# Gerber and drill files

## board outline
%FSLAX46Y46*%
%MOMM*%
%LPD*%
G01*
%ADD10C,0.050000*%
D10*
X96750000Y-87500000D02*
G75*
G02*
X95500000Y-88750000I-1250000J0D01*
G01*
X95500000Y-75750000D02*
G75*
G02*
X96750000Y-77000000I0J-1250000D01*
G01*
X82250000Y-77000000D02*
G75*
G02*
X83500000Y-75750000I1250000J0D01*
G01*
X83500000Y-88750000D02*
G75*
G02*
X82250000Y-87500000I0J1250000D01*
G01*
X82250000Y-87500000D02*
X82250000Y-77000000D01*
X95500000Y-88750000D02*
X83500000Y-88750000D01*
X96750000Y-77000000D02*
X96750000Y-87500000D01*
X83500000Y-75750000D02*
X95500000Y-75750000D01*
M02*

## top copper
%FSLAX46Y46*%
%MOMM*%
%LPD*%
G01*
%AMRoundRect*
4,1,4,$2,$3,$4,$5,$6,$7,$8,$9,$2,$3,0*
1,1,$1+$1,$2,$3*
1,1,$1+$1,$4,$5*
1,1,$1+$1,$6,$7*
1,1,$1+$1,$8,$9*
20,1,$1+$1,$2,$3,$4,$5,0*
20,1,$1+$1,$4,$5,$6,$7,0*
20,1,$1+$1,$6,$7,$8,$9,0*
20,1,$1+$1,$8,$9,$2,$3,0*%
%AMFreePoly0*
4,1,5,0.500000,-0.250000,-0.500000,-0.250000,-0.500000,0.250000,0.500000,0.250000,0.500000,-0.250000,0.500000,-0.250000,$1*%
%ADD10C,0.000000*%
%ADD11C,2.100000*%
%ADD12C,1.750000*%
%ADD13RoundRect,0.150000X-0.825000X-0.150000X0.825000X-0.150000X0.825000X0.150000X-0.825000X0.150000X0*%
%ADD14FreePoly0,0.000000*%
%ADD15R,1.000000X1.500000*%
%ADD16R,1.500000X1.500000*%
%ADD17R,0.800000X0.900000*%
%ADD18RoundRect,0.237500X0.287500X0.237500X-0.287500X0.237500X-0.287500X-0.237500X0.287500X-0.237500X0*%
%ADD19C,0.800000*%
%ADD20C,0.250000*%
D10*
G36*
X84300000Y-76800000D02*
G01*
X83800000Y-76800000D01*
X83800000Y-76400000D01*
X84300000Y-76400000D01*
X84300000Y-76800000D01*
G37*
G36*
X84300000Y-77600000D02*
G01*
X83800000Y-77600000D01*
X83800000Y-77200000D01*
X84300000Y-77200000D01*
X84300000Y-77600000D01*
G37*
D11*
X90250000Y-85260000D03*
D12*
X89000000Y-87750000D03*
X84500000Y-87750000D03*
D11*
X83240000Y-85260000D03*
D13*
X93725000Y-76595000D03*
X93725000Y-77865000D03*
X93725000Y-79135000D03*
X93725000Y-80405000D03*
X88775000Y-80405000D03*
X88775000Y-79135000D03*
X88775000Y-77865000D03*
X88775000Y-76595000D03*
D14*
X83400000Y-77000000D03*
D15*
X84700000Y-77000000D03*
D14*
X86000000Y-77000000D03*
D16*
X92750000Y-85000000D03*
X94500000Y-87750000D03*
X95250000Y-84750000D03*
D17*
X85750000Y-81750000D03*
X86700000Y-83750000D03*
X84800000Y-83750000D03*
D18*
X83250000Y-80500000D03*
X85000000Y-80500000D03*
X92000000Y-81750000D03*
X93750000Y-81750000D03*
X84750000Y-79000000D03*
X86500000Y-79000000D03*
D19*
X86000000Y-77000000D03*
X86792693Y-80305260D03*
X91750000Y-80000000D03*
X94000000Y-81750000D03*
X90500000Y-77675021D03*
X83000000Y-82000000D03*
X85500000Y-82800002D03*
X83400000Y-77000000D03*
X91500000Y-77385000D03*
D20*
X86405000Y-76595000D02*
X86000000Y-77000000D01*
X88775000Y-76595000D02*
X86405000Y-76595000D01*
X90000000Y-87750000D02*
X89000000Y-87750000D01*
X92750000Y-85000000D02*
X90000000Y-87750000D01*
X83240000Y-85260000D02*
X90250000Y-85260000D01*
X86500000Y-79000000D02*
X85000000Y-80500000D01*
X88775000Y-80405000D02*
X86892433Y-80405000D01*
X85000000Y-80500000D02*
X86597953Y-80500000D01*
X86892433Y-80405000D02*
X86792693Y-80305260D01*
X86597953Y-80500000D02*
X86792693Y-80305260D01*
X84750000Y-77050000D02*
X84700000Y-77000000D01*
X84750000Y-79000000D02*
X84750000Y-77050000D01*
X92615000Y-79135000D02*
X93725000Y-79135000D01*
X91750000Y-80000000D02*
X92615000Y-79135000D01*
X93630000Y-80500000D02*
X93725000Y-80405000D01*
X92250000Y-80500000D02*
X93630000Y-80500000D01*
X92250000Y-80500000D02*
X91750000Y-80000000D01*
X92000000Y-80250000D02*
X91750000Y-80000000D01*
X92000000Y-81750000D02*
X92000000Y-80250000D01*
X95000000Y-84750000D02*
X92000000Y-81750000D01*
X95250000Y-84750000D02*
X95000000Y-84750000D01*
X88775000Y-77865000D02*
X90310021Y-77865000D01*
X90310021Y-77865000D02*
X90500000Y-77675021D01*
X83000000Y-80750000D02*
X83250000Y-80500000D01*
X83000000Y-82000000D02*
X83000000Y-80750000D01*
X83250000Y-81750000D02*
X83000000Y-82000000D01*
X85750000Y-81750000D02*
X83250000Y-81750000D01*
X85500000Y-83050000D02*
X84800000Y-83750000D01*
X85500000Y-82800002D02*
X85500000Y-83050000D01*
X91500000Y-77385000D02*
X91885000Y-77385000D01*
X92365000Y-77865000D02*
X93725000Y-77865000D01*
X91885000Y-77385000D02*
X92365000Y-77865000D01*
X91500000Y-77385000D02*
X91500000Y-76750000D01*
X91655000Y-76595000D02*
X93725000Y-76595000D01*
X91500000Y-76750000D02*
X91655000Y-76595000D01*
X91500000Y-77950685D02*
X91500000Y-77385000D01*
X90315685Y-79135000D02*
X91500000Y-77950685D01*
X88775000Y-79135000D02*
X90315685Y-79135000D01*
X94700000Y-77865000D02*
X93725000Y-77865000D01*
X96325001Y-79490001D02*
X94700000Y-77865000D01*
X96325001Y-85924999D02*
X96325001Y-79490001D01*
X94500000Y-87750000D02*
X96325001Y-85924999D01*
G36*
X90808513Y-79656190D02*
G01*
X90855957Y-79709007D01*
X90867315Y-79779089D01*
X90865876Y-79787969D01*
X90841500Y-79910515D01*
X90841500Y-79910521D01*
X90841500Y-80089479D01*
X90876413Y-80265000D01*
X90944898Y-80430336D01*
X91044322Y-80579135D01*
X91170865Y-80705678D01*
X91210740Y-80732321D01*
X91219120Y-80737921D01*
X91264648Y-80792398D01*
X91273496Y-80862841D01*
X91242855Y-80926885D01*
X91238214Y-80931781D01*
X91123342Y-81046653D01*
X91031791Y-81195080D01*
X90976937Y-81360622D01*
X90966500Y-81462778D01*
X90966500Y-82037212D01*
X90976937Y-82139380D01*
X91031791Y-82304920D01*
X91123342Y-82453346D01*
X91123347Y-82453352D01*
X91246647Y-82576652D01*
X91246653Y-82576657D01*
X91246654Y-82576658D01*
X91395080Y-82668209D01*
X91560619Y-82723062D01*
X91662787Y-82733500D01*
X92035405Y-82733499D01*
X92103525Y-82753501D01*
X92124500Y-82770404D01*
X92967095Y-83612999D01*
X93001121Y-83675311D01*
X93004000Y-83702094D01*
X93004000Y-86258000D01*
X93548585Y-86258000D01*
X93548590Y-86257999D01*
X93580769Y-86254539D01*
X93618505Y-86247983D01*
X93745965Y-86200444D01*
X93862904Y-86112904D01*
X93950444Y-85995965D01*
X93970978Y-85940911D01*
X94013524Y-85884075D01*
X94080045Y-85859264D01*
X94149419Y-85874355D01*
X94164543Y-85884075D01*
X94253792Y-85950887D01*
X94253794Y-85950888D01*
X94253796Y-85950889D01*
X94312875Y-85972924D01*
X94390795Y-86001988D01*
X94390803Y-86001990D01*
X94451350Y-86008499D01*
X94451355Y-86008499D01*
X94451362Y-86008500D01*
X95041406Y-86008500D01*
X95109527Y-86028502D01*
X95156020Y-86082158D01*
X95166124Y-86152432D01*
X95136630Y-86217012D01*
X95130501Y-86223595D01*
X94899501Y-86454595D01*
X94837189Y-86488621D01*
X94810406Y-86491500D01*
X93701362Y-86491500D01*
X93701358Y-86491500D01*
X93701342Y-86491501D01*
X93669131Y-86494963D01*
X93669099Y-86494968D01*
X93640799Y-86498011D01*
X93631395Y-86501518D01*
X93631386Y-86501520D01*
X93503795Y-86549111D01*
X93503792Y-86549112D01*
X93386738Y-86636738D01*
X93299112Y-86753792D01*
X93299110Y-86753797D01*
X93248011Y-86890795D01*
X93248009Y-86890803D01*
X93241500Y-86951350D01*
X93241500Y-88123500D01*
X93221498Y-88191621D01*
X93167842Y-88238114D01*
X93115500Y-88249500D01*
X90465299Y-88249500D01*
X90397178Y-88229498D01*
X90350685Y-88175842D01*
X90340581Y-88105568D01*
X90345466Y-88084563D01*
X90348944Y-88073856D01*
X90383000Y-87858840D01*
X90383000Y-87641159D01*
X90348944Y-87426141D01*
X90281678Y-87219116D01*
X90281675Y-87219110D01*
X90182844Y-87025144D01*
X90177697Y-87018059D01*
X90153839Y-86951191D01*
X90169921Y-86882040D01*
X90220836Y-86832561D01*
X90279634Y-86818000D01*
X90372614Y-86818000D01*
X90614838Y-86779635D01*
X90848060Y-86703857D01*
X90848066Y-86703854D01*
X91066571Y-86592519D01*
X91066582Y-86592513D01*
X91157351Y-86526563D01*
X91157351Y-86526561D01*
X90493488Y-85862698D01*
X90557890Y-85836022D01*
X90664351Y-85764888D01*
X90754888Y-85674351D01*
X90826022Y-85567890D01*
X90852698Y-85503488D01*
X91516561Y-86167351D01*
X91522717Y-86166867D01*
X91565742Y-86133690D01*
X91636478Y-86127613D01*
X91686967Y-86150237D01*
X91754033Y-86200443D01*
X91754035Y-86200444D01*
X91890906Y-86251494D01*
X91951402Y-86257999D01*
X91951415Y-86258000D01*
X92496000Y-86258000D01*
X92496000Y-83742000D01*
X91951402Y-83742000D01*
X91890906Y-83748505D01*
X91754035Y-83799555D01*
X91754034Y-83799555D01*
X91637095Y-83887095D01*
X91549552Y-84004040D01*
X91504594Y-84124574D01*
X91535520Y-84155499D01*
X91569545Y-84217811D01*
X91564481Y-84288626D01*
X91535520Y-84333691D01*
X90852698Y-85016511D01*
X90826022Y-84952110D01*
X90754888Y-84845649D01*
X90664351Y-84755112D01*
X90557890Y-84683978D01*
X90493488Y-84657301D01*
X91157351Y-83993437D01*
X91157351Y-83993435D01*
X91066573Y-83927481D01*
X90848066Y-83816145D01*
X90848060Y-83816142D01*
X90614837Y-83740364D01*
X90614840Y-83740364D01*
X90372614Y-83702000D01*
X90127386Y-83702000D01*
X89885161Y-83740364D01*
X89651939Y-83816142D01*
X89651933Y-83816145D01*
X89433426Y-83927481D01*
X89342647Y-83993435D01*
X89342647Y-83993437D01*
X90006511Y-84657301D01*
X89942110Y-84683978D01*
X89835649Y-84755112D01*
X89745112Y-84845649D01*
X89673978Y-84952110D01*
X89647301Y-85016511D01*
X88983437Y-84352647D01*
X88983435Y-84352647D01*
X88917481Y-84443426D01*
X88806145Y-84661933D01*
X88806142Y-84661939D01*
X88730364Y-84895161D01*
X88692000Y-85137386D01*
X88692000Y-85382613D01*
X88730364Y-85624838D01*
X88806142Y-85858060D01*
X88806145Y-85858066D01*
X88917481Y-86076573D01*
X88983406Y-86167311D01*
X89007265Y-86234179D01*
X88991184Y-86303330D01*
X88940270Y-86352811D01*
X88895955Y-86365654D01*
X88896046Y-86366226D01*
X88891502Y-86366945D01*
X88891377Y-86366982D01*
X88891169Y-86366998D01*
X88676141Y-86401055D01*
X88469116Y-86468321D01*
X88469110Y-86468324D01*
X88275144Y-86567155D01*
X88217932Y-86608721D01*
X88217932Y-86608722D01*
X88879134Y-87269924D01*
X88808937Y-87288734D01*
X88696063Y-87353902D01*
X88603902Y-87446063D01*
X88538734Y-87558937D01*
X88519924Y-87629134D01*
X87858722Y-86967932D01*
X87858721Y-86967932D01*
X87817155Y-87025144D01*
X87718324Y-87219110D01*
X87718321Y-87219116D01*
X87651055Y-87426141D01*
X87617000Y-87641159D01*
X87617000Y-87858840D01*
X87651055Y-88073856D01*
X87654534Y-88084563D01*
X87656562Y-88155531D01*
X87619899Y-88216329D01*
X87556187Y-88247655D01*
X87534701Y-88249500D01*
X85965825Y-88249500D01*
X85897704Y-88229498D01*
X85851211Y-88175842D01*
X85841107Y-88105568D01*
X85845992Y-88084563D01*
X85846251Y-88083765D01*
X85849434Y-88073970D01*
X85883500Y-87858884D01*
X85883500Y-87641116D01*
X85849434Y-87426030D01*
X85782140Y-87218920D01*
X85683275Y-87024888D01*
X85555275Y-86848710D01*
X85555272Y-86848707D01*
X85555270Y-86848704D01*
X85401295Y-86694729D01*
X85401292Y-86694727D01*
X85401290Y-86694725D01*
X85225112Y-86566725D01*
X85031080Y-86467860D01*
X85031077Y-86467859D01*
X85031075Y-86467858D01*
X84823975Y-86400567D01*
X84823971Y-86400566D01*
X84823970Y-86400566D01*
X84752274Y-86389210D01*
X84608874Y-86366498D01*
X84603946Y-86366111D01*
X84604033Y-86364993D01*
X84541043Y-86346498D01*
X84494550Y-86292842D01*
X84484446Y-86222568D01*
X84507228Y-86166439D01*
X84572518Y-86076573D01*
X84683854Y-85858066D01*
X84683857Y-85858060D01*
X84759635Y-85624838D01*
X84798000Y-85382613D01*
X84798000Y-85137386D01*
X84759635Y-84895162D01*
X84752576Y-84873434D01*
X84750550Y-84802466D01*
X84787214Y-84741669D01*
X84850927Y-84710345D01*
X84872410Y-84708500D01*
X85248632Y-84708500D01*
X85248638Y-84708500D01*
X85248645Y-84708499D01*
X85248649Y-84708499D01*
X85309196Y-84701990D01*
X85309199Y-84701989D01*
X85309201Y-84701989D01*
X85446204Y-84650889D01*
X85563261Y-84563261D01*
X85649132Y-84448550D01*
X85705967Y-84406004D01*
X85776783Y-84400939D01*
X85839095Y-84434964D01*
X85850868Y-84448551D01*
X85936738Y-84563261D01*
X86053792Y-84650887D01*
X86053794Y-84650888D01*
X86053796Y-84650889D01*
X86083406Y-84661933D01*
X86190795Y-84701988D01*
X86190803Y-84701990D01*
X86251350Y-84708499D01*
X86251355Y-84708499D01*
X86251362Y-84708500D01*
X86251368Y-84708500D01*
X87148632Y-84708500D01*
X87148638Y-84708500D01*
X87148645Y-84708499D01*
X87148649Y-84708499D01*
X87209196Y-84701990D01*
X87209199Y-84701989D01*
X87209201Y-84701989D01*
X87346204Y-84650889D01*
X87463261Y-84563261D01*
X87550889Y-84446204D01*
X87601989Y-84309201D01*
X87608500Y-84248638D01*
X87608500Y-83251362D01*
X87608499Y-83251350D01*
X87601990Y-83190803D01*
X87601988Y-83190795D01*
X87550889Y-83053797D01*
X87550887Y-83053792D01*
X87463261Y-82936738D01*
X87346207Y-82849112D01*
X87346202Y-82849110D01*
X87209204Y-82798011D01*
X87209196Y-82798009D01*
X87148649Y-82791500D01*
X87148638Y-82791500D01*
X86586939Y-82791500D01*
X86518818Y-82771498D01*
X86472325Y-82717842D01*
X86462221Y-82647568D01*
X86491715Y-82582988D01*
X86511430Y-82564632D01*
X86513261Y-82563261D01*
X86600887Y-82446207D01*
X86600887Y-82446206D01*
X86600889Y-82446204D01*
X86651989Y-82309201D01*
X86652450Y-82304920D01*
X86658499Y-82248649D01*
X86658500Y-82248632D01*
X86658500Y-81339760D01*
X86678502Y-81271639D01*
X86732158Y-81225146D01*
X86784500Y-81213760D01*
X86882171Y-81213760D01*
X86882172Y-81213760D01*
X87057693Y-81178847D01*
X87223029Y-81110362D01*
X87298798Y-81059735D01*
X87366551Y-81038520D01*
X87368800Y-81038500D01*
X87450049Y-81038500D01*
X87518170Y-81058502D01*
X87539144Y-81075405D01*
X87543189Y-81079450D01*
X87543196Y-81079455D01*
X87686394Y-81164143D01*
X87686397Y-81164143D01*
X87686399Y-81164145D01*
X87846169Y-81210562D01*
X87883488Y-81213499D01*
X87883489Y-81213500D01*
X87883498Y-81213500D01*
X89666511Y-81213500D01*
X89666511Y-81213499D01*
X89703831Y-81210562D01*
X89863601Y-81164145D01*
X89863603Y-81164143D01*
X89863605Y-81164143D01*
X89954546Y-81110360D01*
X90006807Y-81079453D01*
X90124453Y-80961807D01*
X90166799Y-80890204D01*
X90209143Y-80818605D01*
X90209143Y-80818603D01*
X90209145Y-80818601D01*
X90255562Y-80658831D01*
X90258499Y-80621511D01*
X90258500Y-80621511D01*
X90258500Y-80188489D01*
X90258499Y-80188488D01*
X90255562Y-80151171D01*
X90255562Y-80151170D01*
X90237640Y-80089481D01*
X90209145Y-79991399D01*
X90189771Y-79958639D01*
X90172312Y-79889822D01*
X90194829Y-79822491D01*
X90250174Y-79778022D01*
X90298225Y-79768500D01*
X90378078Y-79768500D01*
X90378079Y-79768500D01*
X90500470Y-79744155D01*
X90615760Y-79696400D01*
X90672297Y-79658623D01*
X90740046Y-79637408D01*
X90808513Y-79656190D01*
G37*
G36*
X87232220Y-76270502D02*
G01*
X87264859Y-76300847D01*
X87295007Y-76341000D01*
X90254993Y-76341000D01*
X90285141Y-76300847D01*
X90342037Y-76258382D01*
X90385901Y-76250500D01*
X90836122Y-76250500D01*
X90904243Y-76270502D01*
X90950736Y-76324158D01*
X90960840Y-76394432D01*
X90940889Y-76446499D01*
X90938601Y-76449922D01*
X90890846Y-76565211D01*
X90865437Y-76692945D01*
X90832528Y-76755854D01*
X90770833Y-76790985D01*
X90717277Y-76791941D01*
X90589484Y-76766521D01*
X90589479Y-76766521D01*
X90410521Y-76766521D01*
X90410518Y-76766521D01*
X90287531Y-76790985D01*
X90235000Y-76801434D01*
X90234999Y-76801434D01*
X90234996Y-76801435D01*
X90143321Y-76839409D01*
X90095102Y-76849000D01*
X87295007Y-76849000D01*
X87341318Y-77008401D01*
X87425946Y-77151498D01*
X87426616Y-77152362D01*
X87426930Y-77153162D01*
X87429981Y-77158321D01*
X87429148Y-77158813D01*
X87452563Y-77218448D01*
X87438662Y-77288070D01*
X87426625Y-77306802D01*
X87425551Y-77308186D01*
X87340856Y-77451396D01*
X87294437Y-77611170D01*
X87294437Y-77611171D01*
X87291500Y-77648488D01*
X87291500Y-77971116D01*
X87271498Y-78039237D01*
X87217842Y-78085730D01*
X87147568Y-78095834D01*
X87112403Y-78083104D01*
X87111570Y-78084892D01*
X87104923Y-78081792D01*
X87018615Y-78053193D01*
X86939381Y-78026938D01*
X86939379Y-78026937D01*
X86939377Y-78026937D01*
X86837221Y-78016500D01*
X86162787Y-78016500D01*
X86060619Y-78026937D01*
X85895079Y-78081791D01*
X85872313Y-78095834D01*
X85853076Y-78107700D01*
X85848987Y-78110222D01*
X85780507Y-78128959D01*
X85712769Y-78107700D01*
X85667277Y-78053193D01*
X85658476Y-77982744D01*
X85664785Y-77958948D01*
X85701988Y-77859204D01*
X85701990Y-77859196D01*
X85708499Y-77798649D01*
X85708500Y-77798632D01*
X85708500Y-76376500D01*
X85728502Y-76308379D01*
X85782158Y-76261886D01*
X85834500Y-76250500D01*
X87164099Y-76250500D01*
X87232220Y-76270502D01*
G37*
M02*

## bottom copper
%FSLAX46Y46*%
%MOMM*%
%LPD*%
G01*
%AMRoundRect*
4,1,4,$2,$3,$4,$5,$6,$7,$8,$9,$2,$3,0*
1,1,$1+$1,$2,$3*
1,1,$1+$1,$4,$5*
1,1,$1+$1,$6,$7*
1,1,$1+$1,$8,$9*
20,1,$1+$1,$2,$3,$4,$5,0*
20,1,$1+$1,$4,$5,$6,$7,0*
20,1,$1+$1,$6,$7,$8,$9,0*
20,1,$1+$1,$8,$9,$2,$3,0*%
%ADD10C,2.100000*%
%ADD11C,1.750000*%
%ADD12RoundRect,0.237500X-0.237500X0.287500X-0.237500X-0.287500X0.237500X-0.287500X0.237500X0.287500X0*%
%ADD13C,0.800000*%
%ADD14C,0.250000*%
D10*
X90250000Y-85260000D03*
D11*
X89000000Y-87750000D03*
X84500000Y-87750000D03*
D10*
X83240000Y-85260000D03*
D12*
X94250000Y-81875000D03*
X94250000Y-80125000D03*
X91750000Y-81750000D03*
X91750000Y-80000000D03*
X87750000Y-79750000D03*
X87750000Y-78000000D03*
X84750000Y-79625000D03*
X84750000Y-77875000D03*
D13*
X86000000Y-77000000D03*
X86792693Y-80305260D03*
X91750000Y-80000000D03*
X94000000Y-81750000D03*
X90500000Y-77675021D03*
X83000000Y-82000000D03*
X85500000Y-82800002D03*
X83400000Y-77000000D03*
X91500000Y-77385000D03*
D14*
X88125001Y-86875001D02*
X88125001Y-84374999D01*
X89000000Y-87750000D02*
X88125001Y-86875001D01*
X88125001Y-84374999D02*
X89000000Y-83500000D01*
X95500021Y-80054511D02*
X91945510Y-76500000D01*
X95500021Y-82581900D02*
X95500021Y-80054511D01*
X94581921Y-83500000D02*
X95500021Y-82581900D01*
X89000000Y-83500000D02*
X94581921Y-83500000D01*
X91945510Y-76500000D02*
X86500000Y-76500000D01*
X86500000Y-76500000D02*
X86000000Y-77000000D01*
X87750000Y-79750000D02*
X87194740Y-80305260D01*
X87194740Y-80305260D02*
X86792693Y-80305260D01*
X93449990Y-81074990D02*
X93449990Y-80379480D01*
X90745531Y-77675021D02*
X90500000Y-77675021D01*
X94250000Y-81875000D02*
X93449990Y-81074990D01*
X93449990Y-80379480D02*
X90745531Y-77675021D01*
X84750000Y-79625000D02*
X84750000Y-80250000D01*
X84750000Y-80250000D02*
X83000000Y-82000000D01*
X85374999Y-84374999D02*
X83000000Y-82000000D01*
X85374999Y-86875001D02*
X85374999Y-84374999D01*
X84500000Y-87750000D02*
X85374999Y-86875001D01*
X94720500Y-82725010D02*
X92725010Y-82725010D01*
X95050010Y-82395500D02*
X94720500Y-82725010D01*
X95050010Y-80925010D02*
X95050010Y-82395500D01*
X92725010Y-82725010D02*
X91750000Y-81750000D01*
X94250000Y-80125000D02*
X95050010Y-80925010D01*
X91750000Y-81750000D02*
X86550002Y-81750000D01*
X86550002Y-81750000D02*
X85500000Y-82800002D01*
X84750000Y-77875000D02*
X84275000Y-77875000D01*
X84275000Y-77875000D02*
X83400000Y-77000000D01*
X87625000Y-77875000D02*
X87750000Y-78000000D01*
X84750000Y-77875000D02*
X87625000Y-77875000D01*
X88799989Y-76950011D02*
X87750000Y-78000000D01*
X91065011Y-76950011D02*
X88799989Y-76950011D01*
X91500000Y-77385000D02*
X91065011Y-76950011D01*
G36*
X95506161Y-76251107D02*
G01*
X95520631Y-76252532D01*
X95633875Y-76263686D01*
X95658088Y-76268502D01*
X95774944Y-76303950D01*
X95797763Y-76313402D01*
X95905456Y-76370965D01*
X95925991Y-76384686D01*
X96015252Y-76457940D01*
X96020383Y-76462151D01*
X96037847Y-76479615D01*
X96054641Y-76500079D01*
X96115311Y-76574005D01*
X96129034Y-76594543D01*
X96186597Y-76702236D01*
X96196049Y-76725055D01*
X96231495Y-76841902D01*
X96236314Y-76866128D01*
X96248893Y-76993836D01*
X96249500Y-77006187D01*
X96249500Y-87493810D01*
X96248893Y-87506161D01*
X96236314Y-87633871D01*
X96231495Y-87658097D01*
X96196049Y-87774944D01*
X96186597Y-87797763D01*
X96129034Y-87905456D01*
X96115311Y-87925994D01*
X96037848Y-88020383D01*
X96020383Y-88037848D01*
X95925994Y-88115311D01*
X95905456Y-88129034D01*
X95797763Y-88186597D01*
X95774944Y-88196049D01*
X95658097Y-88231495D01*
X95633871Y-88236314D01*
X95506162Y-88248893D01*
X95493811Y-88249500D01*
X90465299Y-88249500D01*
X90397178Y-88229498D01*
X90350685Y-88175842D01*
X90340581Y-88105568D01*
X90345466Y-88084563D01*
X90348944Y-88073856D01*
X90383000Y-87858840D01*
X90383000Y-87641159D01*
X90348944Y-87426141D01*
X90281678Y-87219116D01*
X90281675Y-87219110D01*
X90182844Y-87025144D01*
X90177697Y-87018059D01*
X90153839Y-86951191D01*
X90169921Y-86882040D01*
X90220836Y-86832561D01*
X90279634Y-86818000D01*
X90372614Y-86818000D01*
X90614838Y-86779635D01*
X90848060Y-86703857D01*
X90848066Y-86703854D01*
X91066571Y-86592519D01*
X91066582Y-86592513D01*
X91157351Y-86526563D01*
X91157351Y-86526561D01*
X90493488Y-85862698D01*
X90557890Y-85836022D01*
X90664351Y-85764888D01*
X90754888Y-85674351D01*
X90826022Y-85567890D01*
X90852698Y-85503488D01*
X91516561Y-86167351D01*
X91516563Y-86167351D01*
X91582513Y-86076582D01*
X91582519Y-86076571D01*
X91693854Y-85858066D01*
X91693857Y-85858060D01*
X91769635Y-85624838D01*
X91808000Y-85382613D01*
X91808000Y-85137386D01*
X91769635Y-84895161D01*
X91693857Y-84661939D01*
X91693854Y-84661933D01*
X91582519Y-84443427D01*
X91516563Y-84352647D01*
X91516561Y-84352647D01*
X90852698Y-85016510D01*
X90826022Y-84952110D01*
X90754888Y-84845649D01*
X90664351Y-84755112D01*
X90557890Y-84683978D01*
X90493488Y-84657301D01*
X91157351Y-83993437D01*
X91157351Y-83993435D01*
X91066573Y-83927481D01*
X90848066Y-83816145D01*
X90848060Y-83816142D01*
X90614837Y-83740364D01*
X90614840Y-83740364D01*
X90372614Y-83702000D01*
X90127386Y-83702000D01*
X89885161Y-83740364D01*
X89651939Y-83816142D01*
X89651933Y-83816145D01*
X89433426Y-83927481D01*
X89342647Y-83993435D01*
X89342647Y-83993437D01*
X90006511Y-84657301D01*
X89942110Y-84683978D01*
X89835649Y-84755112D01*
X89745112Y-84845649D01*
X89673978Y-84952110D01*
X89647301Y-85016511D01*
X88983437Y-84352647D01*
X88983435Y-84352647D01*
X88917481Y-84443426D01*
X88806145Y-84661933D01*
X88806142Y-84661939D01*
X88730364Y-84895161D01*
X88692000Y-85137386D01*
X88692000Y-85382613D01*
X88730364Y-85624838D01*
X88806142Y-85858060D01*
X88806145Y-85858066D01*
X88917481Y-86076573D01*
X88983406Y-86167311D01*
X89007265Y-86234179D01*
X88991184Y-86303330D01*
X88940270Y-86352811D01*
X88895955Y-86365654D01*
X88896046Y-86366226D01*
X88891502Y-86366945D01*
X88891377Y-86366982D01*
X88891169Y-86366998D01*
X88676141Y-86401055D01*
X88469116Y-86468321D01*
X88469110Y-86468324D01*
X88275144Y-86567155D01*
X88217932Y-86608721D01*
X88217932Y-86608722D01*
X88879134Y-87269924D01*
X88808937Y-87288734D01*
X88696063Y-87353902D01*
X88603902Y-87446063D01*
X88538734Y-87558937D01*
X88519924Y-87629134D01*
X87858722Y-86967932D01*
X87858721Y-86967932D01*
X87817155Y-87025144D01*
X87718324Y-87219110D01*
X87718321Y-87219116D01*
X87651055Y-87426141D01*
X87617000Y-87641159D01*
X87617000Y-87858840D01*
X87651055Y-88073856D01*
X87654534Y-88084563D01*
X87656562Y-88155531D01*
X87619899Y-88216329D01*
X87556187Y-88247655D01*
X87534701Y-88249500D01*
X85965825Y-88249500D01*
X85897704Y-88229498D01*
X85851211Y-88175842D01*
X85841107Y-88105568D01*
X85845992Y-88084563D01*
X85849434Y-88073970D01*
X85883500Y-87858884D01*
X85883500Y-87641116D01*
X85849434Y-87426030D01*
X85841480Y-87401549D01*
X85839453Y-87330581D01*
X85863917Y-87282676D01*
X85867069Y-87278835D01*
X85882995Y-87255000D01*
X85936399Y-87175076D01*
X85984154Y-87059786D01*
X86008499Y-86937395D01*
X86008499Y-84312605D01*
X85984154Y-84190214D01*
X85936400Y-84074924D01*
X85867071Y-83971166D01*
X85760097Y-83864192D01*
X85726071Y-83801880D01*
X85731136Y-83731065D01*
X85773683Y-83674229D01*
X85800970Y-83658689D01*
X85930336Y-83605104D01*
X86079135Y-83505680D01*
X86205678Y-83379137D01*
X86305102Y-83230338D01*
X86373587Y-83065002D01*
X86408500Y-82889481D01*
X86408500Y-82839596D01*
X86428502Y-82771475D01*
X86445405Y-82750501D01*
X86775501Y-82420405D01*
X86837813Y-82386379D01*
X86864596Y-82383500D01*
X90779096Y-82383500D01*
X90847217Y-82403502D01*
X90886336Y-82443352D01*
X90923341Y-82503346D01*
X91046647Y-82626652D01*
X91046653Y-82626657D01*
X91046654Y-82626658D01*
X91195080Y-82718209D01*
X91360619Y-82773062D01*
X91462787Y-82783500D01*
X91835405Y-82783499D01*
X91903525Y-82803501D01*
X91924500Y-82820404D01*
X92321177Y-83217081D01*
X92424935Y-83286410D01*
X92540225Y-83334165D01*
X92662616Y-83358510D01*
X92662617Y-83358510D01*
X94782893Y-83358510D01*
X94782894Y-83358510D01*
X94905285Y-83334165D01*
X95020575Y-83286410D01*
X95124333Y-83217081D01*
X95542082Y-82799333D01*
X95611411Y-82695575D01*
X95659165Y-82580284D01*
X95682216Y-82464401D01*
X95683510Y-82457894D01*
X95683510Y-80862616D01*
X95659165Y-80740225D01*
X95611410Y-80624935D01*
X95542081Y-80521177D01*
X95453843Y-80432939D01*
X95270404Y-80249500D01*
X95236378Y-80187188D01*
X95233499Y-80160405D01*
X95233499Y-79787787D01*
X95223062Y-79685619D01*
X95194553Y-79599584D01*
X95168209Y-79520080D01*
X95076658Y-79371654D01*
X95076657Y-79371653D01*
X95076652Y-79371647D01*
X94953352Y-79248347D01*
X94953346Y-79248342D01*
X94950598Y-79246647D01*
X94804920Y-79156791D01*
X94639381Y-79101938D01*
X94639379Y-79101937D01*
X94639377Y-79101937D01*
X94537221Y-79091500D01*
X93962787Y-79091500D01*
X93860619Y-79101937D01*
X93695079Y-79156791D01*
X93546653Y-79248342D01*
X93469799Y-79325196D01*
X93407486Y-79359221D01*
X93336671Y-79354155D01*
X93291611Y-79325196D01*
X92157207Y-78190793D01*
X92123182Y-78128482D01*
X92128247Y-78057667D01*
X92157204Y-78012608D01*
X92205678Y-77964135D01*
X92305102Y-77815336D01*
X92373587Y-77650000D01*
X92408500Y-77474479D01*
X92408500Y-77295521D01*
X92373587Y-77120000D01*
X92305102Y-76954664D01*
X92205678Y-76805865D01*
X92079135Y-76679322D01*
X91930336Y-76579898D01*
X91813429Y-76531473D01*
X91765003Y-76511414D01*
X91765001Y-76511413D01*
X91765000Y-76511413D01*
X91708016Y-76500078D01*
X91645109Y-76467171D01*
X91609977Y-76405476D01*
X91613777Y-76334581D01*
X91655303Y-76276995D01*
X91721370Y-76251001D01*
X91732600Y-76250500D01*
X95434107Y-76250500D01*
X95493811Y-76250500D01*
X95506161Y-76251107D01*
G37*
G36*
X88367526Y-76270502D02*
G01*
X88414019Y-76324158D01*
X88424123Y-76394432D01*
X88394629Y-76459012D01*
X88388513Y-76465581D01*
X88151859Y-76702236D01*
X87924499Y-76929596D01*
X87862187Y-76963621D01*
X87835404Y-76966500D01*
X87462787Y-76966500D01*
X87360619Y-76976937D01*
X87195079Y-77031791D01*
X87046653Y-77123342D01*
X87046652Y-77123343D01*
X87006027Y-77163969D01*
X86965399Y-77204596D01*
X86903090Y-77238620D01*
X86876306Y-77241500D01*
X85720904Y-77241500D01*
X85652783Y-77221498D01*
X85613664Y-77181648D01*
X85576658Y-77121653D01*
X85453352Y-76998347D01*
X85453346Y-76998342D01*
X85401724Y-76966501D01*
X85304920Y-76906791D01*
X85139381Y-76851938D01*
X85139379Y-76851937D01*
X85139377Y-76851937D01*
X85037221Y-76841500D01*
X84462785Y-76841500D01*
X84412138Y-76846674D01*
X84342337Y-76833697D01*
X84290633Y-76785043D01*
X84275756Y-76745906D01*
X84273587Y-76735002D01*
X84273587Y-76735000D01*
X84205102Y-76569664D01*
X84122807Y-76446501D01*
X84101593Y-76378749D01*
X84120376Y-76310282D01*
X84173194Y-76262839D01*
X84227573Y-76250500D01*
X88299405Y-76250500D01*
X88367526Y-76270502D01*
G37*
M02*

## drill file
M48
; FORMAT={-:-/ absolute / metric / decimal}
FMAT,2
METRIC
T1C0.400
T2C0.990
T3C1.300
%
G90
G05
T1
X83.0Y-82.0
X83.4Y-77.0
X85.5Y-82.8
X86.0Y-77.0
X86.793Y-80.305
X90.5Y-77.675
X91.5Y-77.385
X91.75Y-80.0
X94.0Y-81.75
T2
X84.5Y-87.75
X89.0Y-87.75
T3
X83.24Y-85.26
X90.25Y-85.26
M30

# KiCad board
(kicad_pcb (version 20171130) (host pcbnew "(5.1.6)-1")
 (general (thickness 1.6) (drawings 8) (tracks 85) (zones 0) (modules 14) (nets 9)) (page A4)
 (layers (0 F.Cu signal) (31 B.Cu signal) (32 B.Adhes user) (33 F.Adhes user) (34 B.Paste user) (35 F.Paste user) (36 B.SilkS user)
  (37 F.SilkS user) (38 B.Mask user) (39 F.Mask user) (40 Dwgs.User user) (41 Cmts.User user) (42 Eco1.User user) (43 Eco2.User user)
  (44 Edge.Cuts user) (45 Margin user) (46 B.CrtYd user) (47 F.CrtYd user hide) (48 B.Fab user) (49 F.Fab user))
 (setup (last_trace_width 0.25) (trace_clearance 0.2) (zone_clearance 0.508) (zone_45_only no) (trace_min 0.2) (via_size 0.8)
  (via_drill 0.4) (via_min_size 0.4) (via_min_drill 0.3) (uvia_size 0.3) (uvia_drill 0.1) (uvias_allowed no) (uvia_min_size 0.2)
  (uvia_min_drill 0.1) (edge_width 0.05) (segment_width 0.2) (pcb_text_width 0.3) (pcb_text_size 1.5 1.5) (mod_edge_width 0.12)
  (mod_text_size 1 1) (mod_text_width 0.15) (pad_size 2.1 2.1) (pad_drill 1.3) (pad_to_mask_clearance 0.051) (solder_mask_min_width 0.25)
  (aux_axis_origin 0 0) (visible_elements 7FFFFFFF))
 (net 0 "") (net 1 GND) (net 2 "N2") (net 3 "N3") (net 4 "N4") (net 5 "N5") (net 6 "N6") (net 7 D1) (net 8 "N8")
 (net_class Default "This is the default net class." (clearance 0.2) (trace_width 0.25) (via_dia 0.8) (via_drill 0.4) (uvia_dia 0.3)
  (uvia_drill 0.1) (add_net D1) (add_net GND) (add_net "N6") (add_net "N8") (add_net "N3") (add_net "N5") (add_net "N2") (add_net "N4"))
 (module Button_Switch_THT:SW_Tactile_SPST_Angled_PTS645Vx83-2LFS (layer F.Cu) (at 89 87.75 180)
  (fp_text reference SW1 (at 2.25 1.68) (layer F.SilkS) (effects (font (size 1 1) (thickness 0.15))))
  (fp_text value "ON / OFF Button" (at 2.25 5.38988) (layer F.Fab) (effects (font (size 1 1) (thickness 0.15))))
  (pad "" thru_hole circle (at -1.25 2.49 180) (size 2.1 2.1) (drill 1.3) (layers *.Cu *.Mask) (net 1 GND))
  (pad 1 thru_hole circle (at 0 0 180) (size 1.75 1.75) (drill 0.99) (layers *.Cu *.Mask) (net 1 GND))
  (pad 2 thru_hole circle (at 4.5 0 180) (size 1.75 1.75) (drill 0.99) (layers *.Cu *.Mask) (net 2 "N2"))
  (pad "" thru_hole circle (at 5.76 2.49 180) (size 2.1 2.1) (drill 1.3) (layers *.Cu *.Mask) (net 1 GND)))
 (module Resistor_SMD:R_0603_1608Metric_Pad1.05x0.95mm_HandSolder (layer B.Cu) (at 94.25 81 270)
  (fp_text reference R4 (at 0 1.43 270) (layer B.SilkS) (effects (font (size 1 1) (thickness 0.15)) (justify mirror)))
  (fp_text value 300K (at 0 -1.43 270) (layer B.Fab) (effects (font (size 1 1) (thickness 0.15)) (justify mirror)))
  (pad 2 smd roundrect (at 0.875 0 270) (size 1.05 0.95) (layers B.Cu B.Paste B.Mask) (roundrect_rratio 0.25) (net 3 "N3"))
  (pad 1 smd roundrect (at -0.875 0 270) (size 1.05 0.95) (layers B.Cu B.Paste B.Mask) (roundrect_rratio 0.25) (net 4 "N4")))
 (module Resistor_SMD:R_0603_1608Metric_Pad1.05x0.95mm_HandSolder (layer B.Cu) (at 91.75 80.875 270)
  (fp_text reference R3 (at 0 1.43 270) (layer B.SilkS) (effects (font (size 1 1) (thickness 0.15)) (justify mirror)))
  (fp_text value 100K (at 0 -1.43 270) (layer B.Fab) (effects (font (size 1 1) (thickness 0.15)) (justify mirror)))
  (pad 2 smd roundrect (at 0.875 0 270) (size 1.05 0.95) (layers B.Cu B.Paste B.Mask) (roundrect_rratio 0.25) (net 4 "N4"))
  (pad 1 smd roundrect (at -0.875 0 270) (size 1.05 0.95) (layers B.Cu B.Paste B.Mask) (roundrect_rratio 0.25) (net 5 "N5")))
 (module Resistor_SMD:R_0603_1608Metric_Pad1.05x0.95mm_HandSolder (layer B.Cu) (at 87.75 78.875 270)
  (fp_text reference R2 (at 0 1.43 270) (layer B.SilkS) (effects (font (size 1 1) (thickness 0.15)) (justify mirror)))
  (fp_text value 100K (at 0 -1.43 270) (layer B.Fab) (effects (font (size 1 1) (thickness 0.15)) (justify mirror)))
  (pad 2 smd roundrect (at 0.875 0 270) (size 1.05 0.95) (layers B.Cu B.Paste B.Mask) (roundrect_rratio 0.25) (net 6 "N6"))
  (pad 1 smd roundrect (at -0.875 0 270) (size 1.05 0.95) (layers B.Cu B.Paste B.Mask) (roundrect_rratio 0.25) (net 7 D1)))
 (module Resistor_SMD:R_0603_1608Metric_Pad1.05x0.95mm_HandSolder (layer B.Cu) (at 84.75 78.75 270)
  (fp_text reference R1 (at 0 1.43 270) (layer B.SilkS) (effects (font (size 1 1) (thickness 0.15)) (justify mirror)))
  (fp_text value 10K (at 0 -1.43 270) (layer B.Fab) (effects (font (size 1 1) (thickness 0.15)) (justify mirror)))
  (pad 2 smd roundrect (at 0.875 0 270) (size 1.05 0.95) (layers B.Cu B.Paste B.Mask) (roundrect_rratio 0.25) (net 2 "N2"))
  (pad 1 smd roundrect (at -0.875 0 270) (size 1.05 0.95) (layers B.Cu B.Paste B.Mask) (roundrect_rratio 0.25) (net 7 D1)))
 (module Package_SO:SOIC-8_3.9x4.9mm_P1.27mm (layer F.Cu) (at 91.25 78.5)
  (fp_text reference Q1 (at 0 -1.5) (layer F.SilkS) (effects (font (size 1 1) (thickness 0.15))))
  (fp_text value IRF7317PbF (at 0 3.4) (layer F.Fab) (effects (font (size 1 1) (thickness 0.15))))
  (pad 8 smd roundrect (at 2.475 -1.905) (size 1.95 0.6) (layers F.Cu F.Paste F.Mask) (roundrect_rratio 0.25) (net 7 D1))
  (pad 7 smd roundrect (at 2.475 -0.635) (size 1.95 0.6) (layers F.Cu F.Paste F.Mask) (roundrect_rratio 0.25) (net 7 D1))
  (pad 6 smd roundrect (at 2.475 0.635) (size 1.95 0.6) (layers F.Cu F.Paste F.Mask) (roundrect_rratio 0.25) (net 5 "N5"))
  (pad 5 smd roundrect (at 2.475 1.905) (size 1.95 0.6) (layers F.Cu F.Paste F.Mask) (roundrect_rratio 0.25) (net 5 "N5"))
  (pad 4 smd roundrect (at -2.475 1.905) (size 1.95 0.6) (layers F.Cu F.Paste F.Mask) (roundrect_rratio 0.25) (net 6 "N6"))
  (pad 3 smd roundrect (at -2.475 0.635) (size 1.95 0.6) (layers F.Cu F.Paste F.Mask) (roundrect_rratio 0.25) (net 7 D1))
  (pad 2 smd roundrect (at -2.475 -0.635) (size 1.95 0.6) (layers F.Cu F.Paste F.Mask) (roundrect_rratio 0.25) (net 3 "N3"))
  (pad 1 smd roundrect (at -2.475 -1.905) (size 1.95 0.6) (layers F.Cu F.Paste F.Mask) (roundrect_rratio 0.25) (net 1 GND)))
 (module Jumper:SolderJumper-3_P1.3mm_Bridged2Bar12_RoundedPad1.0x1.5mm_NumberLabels (layer F.Cu) (at 84.7 77)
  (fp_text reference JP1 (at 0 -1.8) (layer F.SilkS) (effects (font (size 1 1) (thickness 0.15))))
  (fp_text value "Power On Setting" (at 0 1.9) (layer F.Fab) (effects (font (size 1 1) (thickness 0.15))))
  (fp_poly (pts (xy -0.9 -0.6) (xy -0.4 -0.6) (xy -0.4 -0.2) (xy -0.9 -0.2)) (layer F.Cu) (width 0))
  (fp_poly (pts (xy -0.9 0.2) (xy -0.4 0.2) (xy -0.4 0.6) (xy -0.9 0.6)) (layer F.Cu) (width 0))
  (pad 1 smd custom (at -1.3 0) (size 1 0.5) (layers F.Cu F.Mask) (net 7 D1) (zone_connect 2) (options (clearance outline) (anchor rect))
   (primitives))
  (pad 2 smd rect (at 0 0) (size 1 1.5) (layers F.Cu F.Mask) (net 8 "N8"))
  (pad 3 smd custom (at 1.3 0) (size 1 0.5) (layers F.Cu F.Mask) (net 1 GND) (zone_connect 2) (options (clearance outline) (anchor rect))
   (primitives)))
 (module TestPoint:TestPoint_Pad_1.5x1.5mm (layer F.Cu) (at 92.75 85)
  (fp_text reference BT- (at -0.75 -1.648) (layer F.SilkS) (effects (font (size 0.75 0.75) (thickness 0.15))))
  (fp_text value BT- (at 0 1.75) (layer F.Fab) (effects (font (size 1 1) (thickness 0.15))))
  (pad 1 smd rect (at 0 0) (size 1.5 1.5) (layers F.Cu F.Mask) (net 1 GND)))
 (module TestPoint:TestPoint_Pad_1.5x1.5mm (layer F.Cu) (at 94.5 87.75)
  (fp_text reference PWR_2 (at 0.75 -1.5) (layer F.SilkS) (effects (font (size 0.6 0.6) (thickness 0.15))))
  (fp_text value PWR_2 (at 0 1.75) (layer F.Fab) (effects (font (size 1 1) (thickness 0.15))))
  (pad 1 smd rect (at 0 0) (size 1.5 1.5) (layers F.Cu F.Mask) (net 7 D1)))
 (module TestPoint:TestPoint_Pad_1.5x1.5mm (layer F.Cu) (at 95.25 84.75)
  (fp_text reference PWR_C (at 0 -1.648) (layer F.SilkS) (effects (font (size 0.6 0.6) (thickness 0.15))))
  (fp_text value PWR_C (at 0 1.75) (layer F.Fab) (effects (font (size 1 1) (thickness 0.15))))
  (pad 1 smd rect (at 0 0) (size 1.5 1.5) (layers F.Cu F.Mask) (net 5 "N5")))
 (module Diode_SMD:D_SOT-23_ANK (layer F.Cu) (at 85.75 82.75 90)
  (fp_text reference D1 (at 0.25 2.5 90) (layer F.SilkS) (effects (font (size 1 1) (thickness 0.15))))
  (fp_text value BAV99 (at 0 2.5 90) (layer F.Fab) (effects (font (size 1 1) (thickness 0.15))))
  (pad 1 smd rect (at 1 0 90) (size 0.9 0.8) (layers F.Cu F.Paste F.Mask) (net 2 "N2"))
  (pad "" smd rect (at -1 0.95 90) (size 0.9 0.8) (layers F.Cu F.Paste F.Mask))
  (pad 2 smd rect (at -1 -0.95 90) (size 0.9 0.8) (layers F.Cu F.Paste F.Mask) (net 4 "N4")))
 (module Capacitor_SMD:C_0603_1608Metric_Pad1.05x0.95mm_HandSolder (layer F.Cu) (at 84.125 80.5 180)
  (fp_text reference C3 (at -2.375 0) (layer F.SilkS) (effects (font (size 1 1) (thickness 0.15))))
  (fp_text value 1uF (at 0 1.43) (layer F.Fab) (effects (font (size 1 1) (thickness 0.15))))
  (pad 2 smd roundrect (at 0.875 0 180) (size 1.05 0.95) (layers F.Cu F.Paste F.Mask) (roundrect_rratio 0.25) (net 2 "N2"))
  (pad 1 smd roundrect (at -0.875 0 180) (size 1.05 0.95) (layers F.Cu F.Paste F.Mask) (roundrect_rratio 0.25) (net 6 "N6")))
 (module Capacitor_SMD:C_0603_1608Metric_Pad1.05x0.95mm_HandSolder (layer F.Cu) (at 92.875 81.75 180)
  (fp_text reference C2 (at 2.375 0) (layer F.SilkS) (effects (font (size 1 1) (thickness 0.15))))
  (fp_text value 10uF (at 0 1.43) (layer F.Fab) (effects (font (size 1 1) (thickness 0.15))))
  (pad 2 smd roundrect (at 0.875 0 180) (size 1.05 0.95) (layers F.Cu F.Paste F.Mask) (roundrect_rratio 0.25) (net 5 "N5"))
  (pad 1 smd roundrect (at -0.875 0 180) (size 1.05 0.95) (layers F.Cu F.Paste F.Mask) (roundrect_rratio 0.25) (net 3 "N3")))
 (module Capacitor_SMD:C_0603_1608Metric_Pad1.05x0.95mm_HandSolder (layer F.Cu) (at 85.625 79 180)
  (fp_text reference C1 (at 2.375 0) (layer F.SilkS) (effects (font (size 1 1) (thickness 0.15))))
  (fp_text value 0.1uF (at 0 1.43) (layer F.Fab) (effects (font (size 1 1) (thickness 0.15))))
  (pad 2 smd roundrect (at 0.875 0 180) (size 1.05 0.95) (layers F.Cu F.Paste F.Mask) (roundrect_rratio 0.25) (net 8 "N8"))
  (pad 1 smd roundrect (at -0.875 0 180) (size 1.05 0.95) (layers F.Cu F.Paste F.Mask) (roundrect_rratio 0.25) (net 6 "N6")))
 (gr_arc (start 95.5 87.5) (end 95.5 88.75) (angle -90) (layer Edge.Cuts) (width 0.05))
 (gr_arc (start 95.5 77) (end 96.75 77) (angle -90) (layer Edge.Cuts) (width 0.05))
 (gr_arc (start 83.5 77) (end 83.5 75.75) (angle -90) (layer Edge.Cuts) (width 0.05))
 (gr_arc (start 83.5 87.5) (end 82.25 87.5) (angle -90) (layer Edge.Cuts) (width 0.05))
 (gr_line (start 82.25 87.5) (end 82.25 77) (layer Edge.Cuts) (width 0.05))
 (gr_line (start 95.5 88.75) (end 83.5 88.75) (layer Edge.Cuts) (width 0.05))
 (gr_line (start 96.75 77) (end 96.75 87.5) (layer Edge.Cuts) (width 0.05))
 (gr_line (start 83.5 75.75) (end 95.5 75.75) (layer Edge.Cuts) (width 0.05))
 (segment (start 86.405 76.595) (end 86 77) (width 0.25) (layer F.Cu) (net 1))
 (segment (start 88.775 76.595) (end 86.405 76.595) (width 0.25) (layer F.Cu) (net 1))
 (segment (start 88.125001 86.875001) (end 88.125001 84.374999) (width 0.25) (layer B.Cu) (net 1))
 (segment (start 89 87.75) (end 88.125001 86.875001) (width 0.25) (layer B.Cu) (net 1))
 (segment (start 88.125001 84.374999) (end 89 83.5) (width 0.25) (layer B.Cu) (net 1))
 (segment (start 95.500021 80.054511) (end 91.94551 76.5) (width 0.25) (layer B.Cu) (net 1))
 (segment (start 95.500021 82.5819) (end 95.500021 80.054511) (width 0.25) (layer B.Cu) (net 1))
 (segment (start 94.581921 83.5) (end 95.500021 82.5819) (width 0.25) (layer B.Cu) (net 1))
 (segment (start 89 83.5) (end 94.581921 83.5) (width 0.25) (layer B.Cu) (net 1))
 (segment (start 91.94551 76.5) (end 86.5 76.5) (width 0.25) (layer B.Cu) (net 1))
 (via (at 86 77) (size 0.8) (drill 0.4) (layers F.Cu B.Cu) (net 1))
 (segment (start 86.5 76.5) (end 86 77) (width 0.25) (layer B.Cu) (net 1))
 (segment (start 90 87.75) (end 89 87.75) (width 0.25) (layer F.Cu) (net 1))
 (segment (start 92.75 85) (end 90 87.75) (width 0.25) (layer F.Cu) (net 1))
 (segment (start 83.24 85.26) (end 90.25 85.26) (width 0.25) (layer F.Cu) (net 1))
 (segment (start 86.5 79) (end 85 80.5) (width 0.25) (layer F.Cu) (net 6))
 (via (at 86.792693 80.30526) (size 0.8) (drill 0.4) (layers F.Cu B.Cu) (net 6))
 (segment (start 88.775 80.405) (end 86.892433 80.405) (width 0.25) (layer F.Cu) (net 6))
 (segment (start 85 80.5) (end 86.597953 80.5) (width 0.25) (layer F.Cu) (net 6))
 (segment (start 86.892433 80.405) (end 86.792693 80.30526) (width 0.25) (layer F.Cu) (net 6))
 (segment (start 87.75 79.75) (end 87.19474 80.30526) (width 0.25) (layer B.Cu) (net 6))
 (segment (start 87.19474 80.30526) (end 86.792693 80.30526) (width 0.25) (layer B.Cu) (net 6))
 (segment (start 86.597953 80.5) (end 86.792693 80.30526) (width 0.25) (layer F.Cu) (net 6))
 (segment (start 84.75 77.05) (end 84.7 77) (width 0.25) (layer F.Cu) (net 8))
 (segment (start 84.75 79) (end 84.75 77.05) (width 0.25) (layer F.Cu) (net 8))
 (via (at 91.75 80) (size 0.8) (drill 0.4) (layers F.Cu B.Cu) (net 5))
 (segment (start 92.615 79.135) (end 93.725 79.135) (width 0.25) (layer F.Cu) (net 5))
 (segment (start 91.75 80) (end 92.615 79.135) (width 0.25) (layer F.Cu) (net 5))
 (segment (start 93.63 80.5) (end 93.725 80.405) (width 0.25) (layer F.Cu) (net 5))
 (segment (start 92.25 80.5) (end 93.63 80.5) (width 0.25) (layer F.Cu) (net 5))
 (segment (start 92.25 80.5) (end 91.75 80) (width 0.25) (layer F.Cu) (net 5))
 (segment (start 92 80.25) (end 91.75 80) (width 0.25) (layer F.Cu) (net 5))
 (segment (start 92 81.75) (end 92 80.25) (width 0.25) (layer F.Cu) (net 5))
 (segment (start 95 84.75) (end 92 81.75) (width 0.25) (layer F.Cu) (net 5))
 (segment (start 95.25 84.75) (end 95 84.75) (width 0.25) (layer F.Cu) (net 5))
 (via (at 94 81.75) (size 0.8) (drill 0.4) (layers F.Cu B.Cu) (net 3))
 (segment (start 88.775 77.865) (end 90.310021 77.865) (width 0.25) (layer F.Cu) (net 3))
 (segment (start 93.44999 81.07499) (end 93.44999 80.37948) (width 0.25) (layer B.Cu) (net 3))
 (segment (start 90.745531 77.675021) (end 90.5 77.675021) (width 0.25) (layer B.Cu) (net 3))
 (segment (start 90.310021 77.865) (end 90.5 77.675021) (width 0.25) (layer F.Cu) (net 3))
 (segment (start 94.25 81.875) (end 93.44999 81.07499) (width 0.25) (layer B.Cu) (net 3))
 (via (at 90.5 77.675021) (size 0.8) (drill 0.4) (layers F.Cu B.Cu) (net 3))
 (segment (start 93.44999 80.37948) (end 90.745531 77.675021) (width 0.25) (layer B.Cu) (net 3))
 (via (at 83 82) (size 0.8) (drill 0.4) (layers F.Cu B.Cu) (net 2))
 (segment (start 84.75 79.625) (end 84.75 80.25) (width 0.25) (layer B.Cu) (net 2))
 (segment (start 84.75 80.25) (end 83 82) (width 0.25) (layer B.Cu) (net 2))
 (segment (start 83 80.75) (end 83.25 80.5) (width 0.25) (layer F.Cu) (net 2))
 (segment (start 83 82) (end 83 80.75) (width 0.25) (layer F.Cu) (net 2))
 (segment (start 83.25 81.75) (end 83 82) (width 0.25) (layer F.Cu) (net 2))
 (segment (start 85.75 81.75) (end 83.25 81.75) (width 0.25) (layer F.Cu) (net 2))
 (segment (start 85.374999 84.374999) (end 83 82) (width 0.25) (layer B.Cu) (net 2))
 (segment (start 85.374999 86.875001) (end 85.374999 84.374999) (width 0.25) (layer B.Cu) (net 2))
 (segment (start 84.5 87.75) (end 85.374999 86.875001) (width 0.25) (layer B.Cu) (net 2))
 (segment (start 94.7205 82.72501) (end 92.72501 82.72501) (width 0.25) (layer B.Cu) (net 4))
 (segment (start 95.05001 82.3955) (end 94.7205 82.72501) (width 0.25) (layer B.Cu) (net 4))
 (segment (start 95.05001 80.92501) (end 95.05001 82.3955) (width 0.25) (layer B.Cu) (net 4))
 (segment (start 92.72501 82.72501) (end 91.75 81.75) (width 0.25) (layer B.Cu) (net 4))
 (segment (start 94.25 80.125) (end 95.05001 80.92501) (width 0.25) (layer B.Cu) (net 4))
 (segment (start 91.75 81.75) (end 86.550002 81.75) (width 0.25) (layer B.Cu) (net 4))
 (segment (start 86.550002 81.75) (end 85.5 82.800002) (width 0.25) (layer B.Cu) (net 4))
 (via (at 85.5 82.800002) (size 0.8) (drill 0.4) (layers F.Cu B.Cu) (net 4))
 (segment (start 85.5 83.05) (end 84.8 83.75) (width 0.25) (layer F.Cu) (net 4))
 (segment (start 85.5 82.800002) (end 85.5 83.05) (width 0.25) (layer F.Cu) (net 4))
 (segment (start 84.75 77.875) (end 84.275 77.875) (width 0.25) (layer B.Cu) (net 7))
 (via (at 83.4 77) (size 0.8) (drill 0.4) (layers F.Cu B.Cu) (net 7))
 (segment (start 84.275 77.875) (end 83.4 77) (width 0.25) (layer B.Cu) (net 7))
 (segment (start 87.625 77.875) (end 87.75 78) (width 0.25) (layer B.Cu) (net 7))
 (segment (start 84.75 77.875) (end 87.625 77.875) (width 0.25) (layer B.Cu) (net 7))
 (via (at 91.5 77.385) (size 0.8) (drill 0.4) (layers F.Cu B.Cu) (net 7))
 (segment (start 91.5 77.385) (end 91.885 77.385) (width 0.25) (layer F.Cu) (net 7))
 (segment (start 92.365 77.865) (end 93.725 77.865) (width 0.25) (layer F.Cu) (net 7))
 (segment (start 91.885 77.385) (end 92.365 77.865) (width 0.25) (layer F.Cu) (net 7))
 (segment (start 91.5 77.385) (end 91.5 76.75) (width 0.25) (layer F.Cu) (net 7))
 (segment (start 91.655 76.595) (end 93.725 76.595) (width 0.25) (layer F.Cu) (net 7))
 (segment (start 91.5 76.75) (end 91.655 76.595) (width 0.25) (layer F.Cu) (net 7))
 (segment (start 91.5 77.950685) (end 91.5 77.385) (width 0.25) (layer F.Cu) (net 7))
 (segment (start 90.315685 79.135) (end 91.5 77.950685) (width 0.25) (layer F.Cu) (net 7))
 (segment (start 88.775 79.135) (end 90.315685 79.135) (width 0.25) (layer F.Cu) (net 7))
 (segment (start 88.799989 76.950011) (end 87.75 78) (width 0.25) (layer B.Cu) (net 7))
 (segment (start 91.065011 76.950011) (end 88.799989 76.950011) (width 0.25) (layer B.Cu) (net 7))
 (segment (start 91.5 77.385) (end 91.065011 76.950011) (width 0.25) (layer B.Cu) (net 7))
 (segment (start 94.7 77.865) (end 93.725 77.865) (width 0.25) (layer F.Cu) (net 7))
 (segment (start 96.325001 79.490001) (end 94.7 77.865) (width 0.25) (layer F.Cu) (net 7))
 (segment (start 96.325001 85.924999) (end 96.325001 79.490001) (width 0.25) (layer F.Cu) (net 7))
 (segment (start 94.5 87.75) (end 96.325001 85.924999) (width 0.25) (layer F.Cu) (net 7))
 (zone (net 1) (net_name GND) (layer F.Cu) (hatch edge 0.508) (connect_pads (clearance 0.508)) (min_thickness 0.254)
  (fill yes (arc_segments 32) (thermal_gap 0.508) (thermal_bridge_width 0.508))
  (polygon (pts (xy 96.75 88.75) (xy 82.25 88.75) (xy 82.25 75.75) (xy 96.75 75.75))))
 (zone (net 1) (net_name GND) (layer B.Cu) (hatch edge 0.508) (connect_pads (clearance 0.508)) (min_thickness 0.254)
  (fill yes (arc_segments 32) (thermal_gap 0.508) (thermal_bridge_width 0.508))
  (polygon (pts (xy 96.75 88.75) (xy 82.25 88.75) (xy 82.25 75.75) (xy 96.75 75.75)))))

